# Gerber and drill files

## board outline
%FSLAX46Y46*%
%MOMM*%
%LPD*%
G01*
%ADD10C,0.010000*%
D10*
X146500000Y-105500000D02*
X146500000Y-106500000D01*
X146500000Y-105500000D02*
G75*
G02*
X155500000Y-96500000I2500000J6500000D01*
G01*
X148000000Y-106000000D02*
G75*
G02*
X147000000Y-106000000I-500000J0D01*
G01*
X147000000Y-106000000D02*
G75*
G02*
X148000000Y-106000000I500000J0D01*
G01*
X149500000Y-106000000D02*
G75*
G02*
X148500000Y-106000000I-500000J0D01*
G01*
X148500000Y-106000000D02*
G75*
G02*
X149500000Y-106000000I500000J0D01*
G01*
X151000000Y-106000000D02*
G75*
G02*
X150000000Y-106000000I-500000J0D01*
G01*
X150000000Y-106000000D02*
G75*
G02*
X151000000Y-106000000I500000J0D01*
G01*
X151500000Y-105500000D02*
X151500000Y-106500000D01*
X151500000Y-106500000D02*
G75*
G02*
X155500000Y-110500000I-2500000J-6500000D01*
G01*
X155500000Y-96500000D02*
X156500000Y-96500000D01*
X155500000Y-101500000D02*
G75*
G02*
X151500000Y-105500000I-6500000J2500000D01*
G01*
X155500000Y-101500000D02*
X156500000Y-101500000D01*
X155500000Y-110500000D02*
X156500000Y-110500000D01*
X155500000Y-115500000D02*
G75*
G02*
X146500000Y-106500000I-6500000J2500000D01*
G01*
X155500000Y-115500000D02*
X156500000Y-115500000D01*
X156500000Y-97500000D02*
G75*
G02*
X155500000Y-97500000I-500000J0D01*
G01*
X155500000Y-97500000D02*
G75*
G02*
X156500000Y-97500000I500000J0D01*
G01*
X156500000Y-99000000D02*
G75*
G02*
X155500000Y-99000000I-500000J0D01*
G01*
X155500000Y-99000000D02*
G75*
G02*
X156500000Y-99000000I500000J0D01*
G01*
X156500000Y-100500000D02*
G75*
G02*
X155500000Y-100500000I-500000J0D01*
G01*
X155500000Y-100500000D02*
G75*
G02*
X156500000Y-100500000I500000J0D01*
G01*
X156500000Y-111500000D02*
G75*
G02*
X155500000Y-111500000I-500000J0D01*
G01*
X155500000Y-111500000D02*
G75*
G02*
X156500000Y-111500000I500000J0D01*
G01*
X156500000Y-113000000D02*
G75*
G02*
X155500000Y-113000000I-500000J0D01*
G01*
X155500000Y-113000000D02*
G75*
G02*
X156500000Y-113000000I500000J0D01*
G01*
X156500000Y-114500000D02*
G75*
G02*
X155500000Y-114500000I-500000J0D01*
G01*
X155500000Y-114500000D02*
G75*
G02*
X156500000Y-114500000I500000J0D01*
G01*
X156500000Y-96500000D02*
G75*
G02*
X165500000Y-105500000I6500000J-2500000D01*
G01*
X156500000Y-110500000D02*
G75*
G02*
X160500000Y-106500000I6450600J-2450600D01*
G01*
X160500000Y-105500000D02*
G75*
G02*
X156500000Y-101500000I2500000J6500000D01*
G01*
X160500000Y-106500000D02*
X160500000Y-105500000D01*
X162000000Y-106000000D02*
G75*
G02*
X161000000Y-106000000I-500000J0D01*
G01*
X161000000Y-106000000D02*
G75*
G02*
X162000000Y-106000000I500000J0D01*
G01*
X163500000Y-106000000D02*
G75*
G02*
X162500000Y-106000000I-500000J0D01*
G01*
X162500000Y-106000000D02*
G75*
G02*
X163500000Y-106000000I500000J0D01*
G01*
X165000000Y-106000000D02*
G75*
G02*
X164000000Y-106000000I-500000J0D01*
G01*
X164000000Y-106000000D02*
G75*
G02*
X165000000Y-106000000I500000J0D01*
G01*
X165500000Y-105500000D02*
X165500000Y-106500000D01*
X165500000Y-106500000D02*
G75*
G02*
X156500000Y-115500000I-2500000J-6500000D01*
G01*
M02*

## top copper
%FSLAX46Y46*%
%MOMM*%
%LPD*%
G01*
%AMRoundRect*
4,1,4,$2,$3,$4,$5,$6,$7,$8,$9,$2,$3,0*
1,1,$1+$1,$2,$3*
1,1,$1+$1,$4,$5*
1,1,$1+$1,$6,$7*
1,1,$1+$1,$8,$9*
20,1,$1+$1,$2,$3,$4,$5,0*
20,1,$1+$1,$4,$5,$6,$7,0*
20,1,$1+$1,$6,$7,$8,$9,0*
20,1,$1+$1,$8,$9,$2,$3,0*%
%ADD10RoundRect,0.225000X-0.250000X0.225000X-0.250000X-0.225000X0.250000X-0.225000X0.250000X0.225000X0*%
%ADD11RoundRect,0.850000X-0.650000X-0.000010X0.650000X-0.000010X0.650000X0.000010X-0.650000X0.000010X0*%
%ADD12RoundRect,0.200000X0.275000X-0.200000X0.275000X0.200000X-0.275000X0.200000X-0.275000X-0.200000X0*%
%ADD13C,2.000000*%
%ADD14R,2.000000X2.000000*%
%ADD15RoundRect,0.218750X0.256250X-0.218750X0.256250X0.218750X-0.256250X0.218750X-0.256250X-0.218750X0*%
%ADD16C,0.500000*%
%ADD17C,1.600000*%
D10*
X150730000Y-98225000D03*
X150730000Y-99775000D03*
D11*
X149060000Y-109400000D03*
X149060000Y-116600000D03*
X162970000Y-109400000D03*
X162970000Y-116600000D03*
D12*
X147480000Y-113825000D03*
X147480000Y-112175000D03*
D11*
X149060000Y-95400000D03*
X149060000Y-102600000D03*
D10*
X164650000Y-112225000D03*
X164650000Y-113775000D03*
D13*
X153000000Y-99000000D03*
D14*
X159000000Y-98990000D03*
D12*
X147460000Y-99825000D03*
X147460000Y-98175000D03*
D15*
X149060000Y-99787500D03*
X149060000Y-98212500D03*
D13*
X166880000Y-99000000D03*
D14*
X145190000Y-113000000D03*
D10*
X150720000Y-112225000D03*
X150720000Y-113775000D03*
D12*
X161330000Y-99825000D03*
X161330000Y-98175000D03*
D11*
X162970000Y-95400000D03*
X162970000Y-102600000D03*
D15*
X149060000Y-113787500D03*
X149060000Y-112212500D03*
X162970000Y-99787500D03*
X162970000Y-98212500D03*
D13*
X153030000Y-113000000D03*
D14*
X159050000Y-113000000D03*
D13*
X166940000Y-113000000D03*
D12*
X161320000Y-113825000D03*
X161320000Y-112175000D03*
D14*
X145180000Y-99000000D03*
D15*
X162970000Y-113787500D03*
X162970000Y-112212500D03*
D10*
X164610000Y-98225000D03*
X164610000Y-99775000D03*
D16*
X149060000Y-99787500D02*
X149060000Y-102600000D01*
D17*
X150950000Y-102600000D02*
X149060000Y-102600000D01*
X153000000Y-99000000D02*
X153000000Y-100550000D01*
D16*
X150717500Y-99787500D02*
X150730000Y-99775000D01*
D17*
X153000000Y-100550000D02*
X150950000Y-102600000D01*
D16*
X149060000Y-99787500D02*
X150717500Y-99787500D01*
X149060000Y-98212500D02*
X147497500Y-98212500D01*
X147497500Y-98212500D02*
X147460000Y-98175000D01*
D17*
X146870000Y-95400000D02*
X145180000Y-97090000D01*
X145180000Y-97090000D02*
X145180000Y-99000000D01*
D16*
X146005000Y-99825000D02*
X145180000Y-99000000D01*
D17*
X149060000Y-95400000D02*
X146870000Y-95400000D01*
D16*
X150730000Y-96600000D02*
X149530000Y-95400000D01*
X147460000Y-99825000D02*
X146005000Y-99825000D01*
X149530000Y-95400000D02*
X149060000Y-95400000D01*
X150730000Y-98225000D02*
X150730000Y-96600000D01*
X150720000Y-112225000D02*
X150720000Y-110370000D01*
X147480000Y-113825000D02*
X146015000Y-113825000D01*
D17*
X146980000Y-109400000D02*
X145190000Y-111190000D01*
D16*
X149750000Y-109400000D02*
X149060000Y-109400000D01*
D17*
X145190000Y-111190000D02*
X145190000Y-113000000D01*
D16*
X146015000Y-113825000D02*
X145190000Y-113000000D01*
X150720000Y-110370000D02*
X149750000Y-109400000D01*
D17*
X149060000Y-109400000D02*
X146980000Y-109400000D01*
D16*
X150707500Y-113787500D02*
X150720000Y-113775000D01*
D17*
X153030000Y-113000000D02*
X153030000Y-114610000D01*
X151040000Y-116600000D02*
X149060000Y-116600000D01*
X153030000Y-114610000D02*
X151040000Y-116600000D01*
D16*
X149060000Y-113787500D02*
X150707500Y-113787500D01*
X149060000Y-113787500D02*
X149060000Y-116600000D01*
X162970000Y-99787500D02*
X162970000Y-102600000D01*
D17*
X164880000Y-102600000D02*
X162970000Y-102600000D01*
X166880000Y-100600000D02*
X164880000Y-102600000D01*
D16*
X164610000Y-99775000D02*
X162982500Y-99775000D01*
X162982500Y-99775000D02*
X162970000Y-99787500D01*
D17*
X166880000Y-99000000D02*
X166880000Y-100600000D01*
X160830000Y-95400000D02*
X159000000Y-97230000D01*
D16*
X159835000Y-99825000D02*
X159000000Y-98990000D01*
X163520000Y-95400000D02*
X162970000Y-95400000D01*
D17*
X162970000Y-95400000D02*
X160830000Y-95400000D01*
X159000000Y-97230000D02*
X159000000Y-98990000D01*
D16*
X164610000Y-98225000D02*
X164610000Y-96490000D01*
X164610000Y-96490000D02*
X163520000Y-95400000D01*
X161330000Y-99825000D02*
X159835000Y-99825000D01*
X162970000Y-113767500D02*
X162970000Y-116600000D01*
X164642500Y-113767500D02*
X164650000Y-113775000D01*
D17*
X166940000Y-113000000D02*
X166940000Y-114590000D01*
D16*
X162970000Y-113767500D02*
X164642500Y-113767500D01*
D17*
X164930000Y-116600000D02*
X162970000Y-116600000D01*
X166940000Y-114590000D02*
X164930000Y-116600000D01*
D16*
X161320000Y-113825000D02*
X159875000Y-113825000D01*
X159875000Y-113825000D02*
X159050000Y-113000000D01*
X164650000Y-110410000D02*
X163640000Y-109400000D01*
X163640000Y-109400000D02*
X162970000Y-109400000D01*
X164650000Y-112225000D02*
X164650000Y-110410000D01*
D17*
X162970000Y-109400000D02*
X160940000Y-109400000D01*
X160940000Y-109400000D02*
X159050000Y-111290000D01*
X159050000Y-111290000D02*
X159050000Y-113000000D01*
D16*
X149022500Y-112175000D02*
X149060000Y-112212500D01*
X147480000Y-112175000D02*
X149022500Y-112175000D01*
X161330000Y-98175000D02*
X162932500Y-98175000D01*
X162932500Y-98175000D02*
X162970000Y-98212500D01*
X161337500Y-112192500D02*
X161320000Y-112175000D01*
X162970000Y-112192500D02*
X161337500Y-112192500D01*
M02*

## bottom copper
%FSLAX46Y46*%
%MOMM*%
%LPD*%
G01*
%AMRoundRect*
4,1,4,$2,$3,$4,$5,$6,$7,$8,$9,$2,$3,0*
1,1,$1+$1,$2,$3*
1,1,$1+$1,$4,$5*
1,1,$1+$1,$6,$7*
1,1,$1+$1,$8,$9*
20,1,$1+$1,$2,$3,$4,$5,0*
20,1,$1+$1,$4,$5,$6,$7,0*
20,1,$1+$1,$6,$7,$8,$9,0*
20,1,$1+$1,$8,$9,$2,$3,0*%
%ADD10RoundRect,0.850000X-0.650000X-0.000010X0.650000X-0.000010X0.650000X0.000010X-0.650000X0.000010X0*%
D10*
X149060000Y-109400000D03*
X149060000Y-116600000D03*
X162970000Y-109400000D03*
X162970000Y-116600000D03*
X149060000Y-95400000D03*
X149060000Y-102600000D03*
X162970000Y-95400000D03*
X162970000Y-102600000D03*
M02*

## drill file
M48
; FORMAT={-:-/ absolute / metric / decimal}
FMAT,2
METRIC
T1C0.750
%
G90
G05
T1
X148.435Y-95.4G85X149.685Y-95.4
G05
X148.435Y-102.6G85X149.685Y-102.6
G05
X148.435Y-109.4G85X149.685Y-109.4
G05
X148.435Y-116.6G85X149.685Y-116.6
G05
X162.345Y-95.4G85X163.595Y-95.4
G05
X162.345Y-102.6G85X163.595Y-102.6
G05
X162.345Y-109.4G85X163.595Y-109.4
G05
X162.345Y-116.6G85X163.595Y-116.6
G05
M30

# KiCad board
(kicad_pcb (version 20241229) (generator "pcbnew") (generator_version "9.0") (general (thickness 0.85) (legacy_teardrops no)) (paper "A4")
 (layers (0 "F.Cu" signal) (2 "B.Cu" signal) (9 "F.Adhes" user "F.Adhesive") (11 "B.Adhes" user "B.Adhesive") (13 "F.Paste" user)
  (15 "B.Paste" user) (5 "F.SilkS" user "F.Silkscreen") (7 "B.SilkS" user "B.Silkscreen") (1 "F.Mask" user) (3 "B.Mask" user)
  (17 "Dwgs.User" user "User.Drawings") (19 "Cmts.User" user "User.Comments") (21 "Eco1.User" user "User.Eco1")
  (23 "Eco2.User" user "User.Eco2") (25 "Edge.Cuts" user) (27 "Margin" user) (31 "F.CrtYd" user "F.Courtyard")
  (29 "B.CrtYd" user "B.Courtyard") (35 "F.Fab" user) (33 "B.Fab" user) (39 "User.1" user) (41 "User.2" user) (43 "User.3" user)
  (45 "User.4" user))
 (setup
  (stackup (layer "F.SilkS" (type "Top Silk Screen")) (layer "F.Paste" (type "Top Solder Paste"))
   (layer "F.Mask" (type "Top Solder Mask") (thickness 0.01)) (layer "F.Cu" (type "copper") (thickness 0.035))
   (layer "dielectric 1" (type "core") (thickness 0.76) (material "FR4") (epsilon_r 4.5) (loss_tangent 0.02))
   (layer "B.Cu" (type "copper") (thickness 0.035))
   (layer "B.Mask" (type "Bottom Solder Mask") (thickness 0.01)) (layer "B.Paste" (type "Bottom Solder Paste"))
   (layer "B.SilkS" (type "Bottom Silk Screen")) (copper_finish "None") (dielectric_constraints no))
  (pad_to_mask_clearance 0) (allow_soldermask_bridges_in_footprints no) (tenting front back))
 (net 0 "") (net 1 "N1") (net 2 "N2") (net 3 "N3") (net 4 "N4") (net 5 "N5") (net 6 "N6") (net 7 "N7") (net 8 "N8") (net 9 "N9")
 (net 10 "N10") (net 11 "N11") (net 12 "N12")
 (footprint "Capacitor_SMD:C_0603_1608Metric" (layer "F.Cu") (at 150.73 99 -90)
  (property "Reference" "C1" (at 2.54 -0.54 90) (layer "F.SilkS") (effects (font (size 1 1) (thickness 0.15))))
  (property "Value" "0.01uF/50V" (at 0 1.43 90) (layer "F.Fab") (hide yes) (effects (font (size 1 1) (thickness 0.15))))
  (pad "1" smd roundrect (at -0.775 0 270) (size 0.9 0.95) (layers "F.Cu" "F.Mask" "F.Paste") (roundrect_rratio 0.25) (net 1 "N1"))
  (pad "2" smd roundrect (at 0.775 0 270) (size 0.9 0.95) (layers "F.Cu" "F.Mask" "F.Paste") (roundrect_rratio 0.25) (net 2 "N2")))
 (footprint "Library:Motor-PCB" (layer "F.Cu") (at 149.06 113)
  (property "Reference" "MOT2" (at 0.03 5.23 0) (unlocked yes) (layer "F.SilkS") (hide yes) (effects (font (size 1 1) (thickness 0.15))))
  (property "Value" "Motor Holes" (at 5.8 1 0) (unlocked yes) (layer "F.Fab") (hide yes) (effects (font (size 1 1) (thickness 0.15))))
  (pad "1" thru_hole roundrect (at 0 -3.6) (size 3 1.7) (drill oval 2 0.75) (layers "*.Cu" "*.Mask") (remove_unused_layers no)
   (roundrect_rratio 0.5) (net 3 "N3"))
  (pad "2" thru_hole roundrect (at 0 3.6) (size 3 1.7) (drill oval 2 0.75) (layers "*.Cu" "*.Mask") (remove_unused_layers no)
   (roundrect_rratio 0.5) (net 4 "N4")))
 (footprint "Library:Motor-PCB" (layer "F.Cu") (at 162.97 113)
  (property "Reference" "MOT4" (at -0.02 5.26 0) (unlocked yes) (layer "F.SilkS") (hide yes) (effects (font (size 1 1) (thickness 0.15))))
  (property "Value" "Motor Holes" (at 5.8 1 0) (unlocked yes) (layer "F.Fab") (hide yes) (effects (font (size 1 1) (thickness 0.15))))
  (pad "1" thru_hole roundrect (at 0 -3.6) (size 3 1.7) (drill oval 2 0.75) (layers "*.Cu" "*.Mask") (remove_unused_layers no)
   (roundrect_rratio 0.5) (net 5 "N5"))
  (pad "2" thru_hole roundrect (at 0 3.6) (size 3 1.7) (drill oval 2 0.75) (layers "*.Cu" "*.Mask") (remove_unused_layers no)
   (roundrect_rratio 0.5) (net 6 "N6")))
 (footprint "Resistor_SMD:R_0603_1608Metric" (layer "F.Cu") (at 147.48 113 90)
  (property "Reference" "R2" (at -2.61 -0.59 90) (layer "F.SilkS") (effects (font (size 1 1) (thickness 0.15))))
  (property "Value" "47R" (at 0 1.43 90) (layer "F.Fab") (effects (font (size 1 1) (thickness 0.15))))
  (pad "1" smd roundrect (at -0.825 0 90) (size 0.8 0.95) (layers "F.Cu" "F.Mask" "F.Paste") (roundrect_rratio 0.25) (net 3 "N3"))
  (pad "2" smd roundrect (at 0.825 0 90) (size 0.8 0.95) (layers "F.Cu" "F.Mask" "F.Paste") (roundrect_rratio 0.25) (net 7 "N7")))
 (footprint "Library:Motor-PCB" (layer "F.Cu") (at 149.06 99)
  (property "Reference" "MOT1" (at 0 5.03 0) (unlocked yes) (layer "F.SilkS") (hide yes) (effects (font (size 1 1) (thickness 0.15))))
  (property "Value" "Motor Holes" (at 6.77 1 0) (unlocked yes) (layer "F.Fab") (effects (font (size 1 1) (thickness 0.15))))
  (pad "1" thru_hole roundrect (at 0 -3.6) (size 3 1.7) (drill oval 2 0.75) (layers "*.Cu" "*.Mask") (remove_unused_layers no)
   (roundrect_rratio 0.5) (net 1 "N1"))
  (pad "2" thru_hole roundrect (at 0 3.6) (size 3 1.7) (drill oval 2 0.75) (layers "*.Cu" "*.Mask") (remove_unused_layers no)
   (roundrect_rratio 0.5) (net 2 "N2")))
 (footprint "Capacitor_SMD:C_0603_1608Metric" (layer "F.Cu") (at 164.65 113 -90)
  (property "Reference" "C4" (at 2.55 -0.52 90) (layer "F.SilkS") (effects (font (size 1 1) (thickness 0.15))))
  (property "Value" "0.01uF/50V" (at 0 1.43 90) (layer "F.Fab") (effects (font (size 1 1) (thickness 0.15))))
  (pad "1" smd roundrect (at -0.775 0 270) (size 0.9 0.95) (layers "F.Cu" "F.Mask" "F.Paste") (roundrect_rratio 0.25) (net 5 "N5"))
  (pad "2" smd roundrect (at 0.775 0 270) (size 0.9 0.95) (layers "F.Cu" "F.Mask" "F.Paste") (roundrect_rratio 0.25) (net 6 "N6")))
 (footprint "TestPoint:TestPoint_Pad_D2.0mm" (layer "F.Cu") (at 153 99)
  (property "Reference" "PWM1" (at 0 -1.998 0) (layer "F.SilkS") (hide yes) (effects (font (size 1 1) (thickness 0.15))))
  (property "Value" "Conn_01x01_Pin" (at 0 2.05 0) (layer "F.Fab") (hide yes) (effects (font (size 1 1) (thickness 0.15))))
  (pad "1" smd circle (at 0 0) (size 2 2) (layers "F.Cu" "F.Mask") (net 2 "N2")))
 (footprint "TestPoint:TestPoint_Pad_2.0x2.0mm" (layer "F.Cu") (at 159 98.99)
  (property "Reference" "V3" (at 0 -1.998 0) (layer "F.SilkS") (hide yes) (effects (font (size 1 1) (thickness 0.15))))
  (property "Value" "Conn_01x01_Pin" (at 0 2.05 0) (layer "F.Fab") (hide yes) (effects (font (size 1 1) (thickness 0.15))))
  (pad "1" smd rect (at 0 0) (size 2 2) (layers "F.Cu" "F.Mask") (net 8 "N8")))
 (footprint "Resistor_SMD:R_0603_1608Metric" (layer "F.Cu") (at 147.46 99 90)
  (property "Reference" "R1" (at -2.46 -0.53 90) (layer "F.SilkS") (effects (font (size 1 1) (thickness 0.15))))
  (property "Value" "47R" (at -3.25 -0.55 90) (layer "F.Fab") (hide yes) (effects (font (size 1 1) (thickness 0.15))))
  (pad "1" smd roundrect (at -0.825 0 90) (size 0.8 0.95) (layers "F.Cu" "F.Mask" "F.Paste") (roundrect_rratio 0.25) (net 1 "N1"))
  (pad "2" smd roundrect (at 0.825 0 90) (size 0.8 0.95) (layers "F.Cu" "F.Mask" "F.Paste") (roundrect_rratio 0.25) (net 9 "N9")))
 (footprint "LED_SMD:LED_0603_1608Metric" (layer "F.Cu") (at 149.06 99 90)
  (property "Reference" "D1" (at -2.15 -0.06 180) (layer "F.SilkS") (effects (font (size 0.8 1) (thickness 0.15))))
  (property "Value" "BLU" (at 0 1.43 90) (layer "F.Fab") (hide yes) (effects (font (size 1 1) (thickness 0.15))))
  (pad "1" smd roundrect (at -0.7875 0 90) (size 0.875 0.95) (layers "F.Cu" "F.Mask" "F.Paste") (roundrect_rratio 0.25) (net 2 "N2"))
  (pad "2" smd roundrect (at 0.7875 0 90) (size 0.875 0.95) (layers "F.Cu" "F.Mask" "F.Paste") (roundrect_rratio 0.25) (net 9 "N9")))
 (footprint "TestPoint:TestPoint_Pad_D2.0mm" (layer "F.Cu") (at 166.88 99 90)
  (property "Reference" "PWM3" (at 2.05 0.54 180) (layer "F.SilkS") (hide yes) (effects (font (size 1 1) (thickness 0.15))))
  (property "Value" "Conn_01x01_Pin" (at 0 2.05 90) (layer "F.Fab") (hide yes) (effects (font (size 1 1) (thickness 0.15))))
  (pad "1" smd circle (at 0 0 90) (size 2 2) (layers "F.Cu" "F.Mask") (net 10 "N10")))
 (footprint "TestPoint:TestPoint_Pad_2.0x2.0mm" (layer "F.Cu") (at 145.19 113)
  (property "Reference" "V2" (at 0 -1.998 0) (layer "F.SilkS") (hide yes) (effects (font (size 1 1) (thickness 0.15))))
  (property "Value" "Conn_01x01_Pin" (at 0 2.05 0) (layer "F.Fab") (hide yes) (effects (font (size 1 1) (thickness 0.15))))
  (pad "1" smd rect (at 0 0) (size 2 2) (layers "F.Cu" "F.Mask") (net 3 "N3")))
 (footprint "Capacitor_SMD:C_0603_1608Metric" (layer "F.Cu") (at 150.72 113 -90)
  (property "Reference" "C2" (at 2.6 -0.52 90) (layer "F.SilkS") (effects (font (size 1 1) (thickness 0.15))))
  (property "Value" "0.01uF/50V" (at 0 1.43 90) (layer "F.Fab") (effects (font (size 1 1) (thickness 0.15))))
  (pad "1" smd roundrect (at -0.775 0 270) (size 0.9 0.95) (layers "F.Cu" "F.Mask" "F.Paste") (roundrect_rratio 0.25) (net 3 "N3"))
  (pad "2" smd roundrect (at 0.775 0 270) (size 0.9 0.95) (layers "F.Cu" "F.Mask" "F.Paste") (roundrect_rratio 0.25) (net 4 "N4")))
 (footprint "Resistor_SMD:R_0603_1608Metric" (layer "F.Cu") (at 161.33 99 90)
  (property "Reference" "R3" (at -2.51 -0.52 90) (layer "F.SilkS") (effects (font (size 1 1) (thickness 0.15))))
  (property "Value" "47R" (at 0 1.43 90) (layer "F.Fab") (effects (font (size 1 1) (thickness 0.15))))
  (pad "1" smd roundrect (at -0.825 0 90) (size 0.8 0.95) (layers "F.Cu" "F.Mask" "F.Paste") (roundrect_rratio 0.25) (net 8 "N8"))
  (pad "2" smd roundrect (at 0.825 0 90) (size 0.8 0.95) (layers "F.Cu" "F.Mask" "F.Paste") (roundrect_rratio 0.25) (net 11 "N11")))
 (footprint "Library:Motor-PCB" (layer "F.Cu") (at 162.97 99)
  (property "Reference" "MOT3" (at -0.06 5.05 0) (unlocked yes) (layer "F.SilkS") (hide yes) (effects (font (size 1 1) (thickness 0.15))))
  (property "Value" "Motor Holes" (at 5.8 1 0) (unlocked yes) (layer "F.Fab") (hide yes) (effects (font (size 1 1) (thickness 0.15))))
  (pad "1" thru_hole roundrect (at 0 -3.6) (size 3 1.7) (drill oval 2 0.75) (layers "*.Cu" "*.Mask") (remove_unused_layers no)
   (roundrect_rratio 0.5) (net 8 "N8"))
  (pad "2" thru_hole roundrect (at 0 3.6) (size 3 1.7) (drill oval 2 0.75) (layers "*.Cu" "*.Mask") (remove_unused_layers no)
   (roundrect_rratio 0.5) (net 10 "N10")))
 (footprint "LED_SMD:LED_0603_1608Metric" (layer "F.Cu") (at 149.06 113 90)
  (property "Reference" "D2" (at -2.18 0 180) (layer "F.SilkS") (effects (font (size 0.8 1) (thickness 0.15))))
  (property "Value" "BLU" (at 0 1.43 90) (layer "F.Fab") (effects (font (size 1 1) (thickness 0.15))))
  (pad "1" smd roundrect (at -0.7875 0 90) (size 0.875 0.95) (layers "F.Cu" "F.Mask" "F.Paste") (roundrect_rratio 0.25) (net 4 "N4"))
  (pad "2" smd roundrect (at 0.7875 0 90) (size 0.875 0.95) (layers "F.Cu" "F.Mask" "F.Paste") (roundrect_rratio 0.25) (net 7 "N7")))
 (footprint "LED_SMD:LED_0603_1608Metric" (layer "F.Cu") (at 162.97 99 90)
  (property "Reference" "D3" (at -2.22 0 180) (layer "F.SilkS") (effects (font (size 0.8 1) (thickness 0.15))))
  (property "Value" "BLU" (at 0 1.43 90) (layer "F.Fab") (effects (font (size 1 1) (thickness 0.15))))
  (pad "1" smd roundrect (at -0.7875 0 90) (size 0.875 0.95) (layers "F.Cu" "F.Mask" "F.Paste") (roundrect_rratio 0.25) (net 10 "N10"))
  (pad "2" smd roundrect (at 0.7875 0 90) (size 0.875 0.95) (layers "F.Cu" "F.Mask" "F.Paste") (roundrect_rratio 0.25) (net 11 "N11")))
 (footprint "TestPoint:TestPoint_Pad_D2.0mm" (layer "F.Cu") (at 153.03 113)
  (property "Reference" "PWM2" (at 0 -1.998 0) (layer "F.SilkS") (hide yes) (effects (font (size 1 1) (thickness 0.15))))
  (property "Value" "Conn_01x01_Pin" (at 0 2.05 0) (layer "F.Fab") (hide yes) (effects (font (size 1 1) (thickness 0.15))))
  (pad "1" smd circle (at 0 0) (size 2 2) (layers "F.Cu" "F.Mask") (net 4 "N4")))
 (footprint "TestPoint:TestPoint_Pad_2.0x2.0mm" (layer "F.Cu") (at 159.05 113)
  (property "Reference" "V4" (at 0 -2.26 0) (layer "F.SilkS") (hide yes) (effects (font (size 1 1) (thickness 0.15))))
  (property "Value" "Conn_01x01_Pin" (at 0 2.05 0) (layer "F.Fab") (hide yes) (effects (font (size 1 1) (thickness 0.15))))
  (pad "1" smd rect (at 0 0) (size 2 2) (layers "F.Cu" "F.Mask") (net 5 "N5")))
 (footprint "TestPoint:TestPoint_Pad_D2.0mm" (layer "F.Cu") (at 166.94 113)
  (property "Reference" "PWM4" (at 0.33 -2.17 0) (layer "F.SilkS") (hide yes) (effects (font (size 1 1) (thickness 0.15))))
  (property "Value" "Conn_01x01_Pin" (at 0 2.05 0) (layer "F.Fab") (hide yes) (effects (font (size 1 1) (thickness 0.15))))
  (pad "1" smd circle (at 0 0) (size 2 2) (layers "F.Cu" "F.Mask") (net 6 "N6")))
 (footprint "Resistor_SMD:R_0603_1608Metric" (layer "F.Cu") (at 161.32 113 90)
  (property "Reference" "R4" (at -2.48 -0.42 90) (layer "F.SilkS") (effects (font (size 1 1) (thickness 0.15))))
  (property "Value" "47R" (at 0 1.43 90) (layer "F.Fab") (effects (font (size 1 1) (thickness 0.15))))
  (pad "1" smd roundrect (at -0.825 0 90) (size 0.8 0.95) (layers "F.Cu" "F.Mask" "F.Paste") (roundrect_rratio 0.25) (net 5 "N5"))
  (pad "2" smd roundrect (at 0.825 0 90) (size 0.8 0.95) (layers "F.Cu" "F.Mask" "F.Paste") (roundrect_rratio 0.25) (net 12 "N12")))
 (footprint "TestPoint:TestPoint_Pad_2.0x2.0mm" (layer "F.Cu") (at 145.18 99)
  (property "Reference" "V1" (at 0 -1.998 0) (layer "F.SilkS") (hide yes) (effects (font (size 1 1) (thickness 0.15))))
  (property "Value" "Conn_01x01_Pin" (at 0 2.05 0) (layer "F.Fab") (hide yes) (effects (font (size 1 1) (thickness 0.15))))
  (pad "1" smd rect (at 0 0) (size 2 2) (layers "F.Cu" "F.Mask") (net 1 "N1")))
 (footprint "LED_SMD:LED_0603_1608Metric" (layer "F.Cu") (at 162.97 113 90)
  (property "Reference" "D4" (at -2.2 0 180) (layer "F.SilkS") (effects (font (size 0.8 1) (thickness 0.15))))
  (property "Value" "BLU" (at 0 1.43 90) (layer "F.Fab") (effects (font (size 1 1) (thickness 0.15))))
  (pad "1" smd roundrect (at -0.7875 0 90) (size 0.875 0.95) (layers "F.Cu" "F.Mask" "F.Paste") (roundrect_rratio 0.25) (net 6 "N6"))
  (pad "2" smd roundrect (at 0.7875 0 90) (size 0.875 0.95) (layers "F.Cu" "F.Mask" "F.Paste") (roundrect_rratio 0.25) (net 12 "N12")))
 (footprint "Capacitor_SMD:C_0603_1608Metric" (layer "F.Cu") (at 164.61 99 -90)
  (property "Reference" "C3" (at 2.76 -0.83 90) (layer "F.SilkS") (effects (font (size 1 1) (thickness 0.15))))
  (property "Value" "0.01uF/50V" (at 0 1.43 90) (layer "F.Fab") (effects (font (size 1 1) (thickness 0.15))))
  (pad "1" smd roundrect (at -0.775 0 270) (size 0.9 0.95) (layers "F.Cu" "F.Mask" "F.Paste") (roundrect_rratio 0.25) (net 8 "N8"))
  (pad "2" smd roundrect (at 0.775 0 270) (size 0.9 0.95) (layers "F.Cu" "F.Mask" "F.Paste") (roundrect_rratio 0.25) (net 10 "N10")))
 (gr_line (start 146.5 105.5) (end 146.5 106.5) (stroke (width 0.01) (type solid)) (layer "Edge.Cuts"))
 (gr_arc (start 146.5 105.5) (mid 144.075571 94.075571) (end 155.5 96.5) (stroke (width 0.01) (type solid)) (layer "Edge.Cuts"))
 (gr_circle (center 147.5 106) (end 147.5 105.5) (stroke (width 0.01) (type solid)) (fill no) (layer "Edge.Cuts"))
 (gr_circle (center 149 106) (end 149 105.5) (stroke (width 0.01) (type solid)) (fill no) (layer "Edge.Cuts"))
 (gr_circle (center 150.5 106) (end 150.5 105.5) (stroke (width 0.01) (type solid)) (fill no) (layer "Edge.Cuts"))
 (gr_line (start 151.5 105.5) (end 151.5 106.5) (stroke (width 0.01) (type solid)) (layer "Edge.Cuts"))
 (gr_arc (start 151.5 106.5) (mid 153.924429 108.075571) (end 155.5 110.5) (stroke (width 0.01) (type solid)) (layer "Edge.Cuts"))
 (gr_line (start 155.5 96.5) (end 156.5 96.5) (stroke (width 0.01) (type solid)) (layer "Edge.Cuts"))
 (gr_arc (start 155.5 101.5) (mid 153.924429 103.924429) (end 151.5 105.5) (stroke (width 0.01) (type solid)) (layer "Edge.Cuts"))
 (gr_line (start 155.5 101.5) (end 156.5 101.5) (stroke (width 0.01) (type solid)) (layer "Edge.Cuts"))
 (gr_line (start 155.5 110.5) (end 156.5 110.5) (stroke (width 0.01) (type solid)) (layer "Edge.Cuts"))
 (gr_arc (start 155.5 115.5) (mid 144.075571 117.924429) (end 146.5 106.5) (stroke (width 0.01) (type solid)) (layer "Edge.Cuts"))
 (gr_line (start 155.5 115.5) (end 156.5 115.5) (stroke (width 0.01) (type solid)) (layer "Edge.Cuts"))
 (gr_circle (center 156 97.5) (end 155.5 97.5) (stroke (width 0.01) (type solid)) (fill no) (layer "Edge.Cuts"))
 (gr_circle (center 156 99) (end 155.5 99) (stroke (width 0.01) (type solid)) (fill no) (layer "Edge.Cuts"))
 (gr_circle (center 156 100.5) (end 155.5 100.5) (stroke (width 0.01) (type solid)) (fill no) (layer "Edge.Cuts"))
 (gr_circle (center 156 111.5) (end 155.5 111.5) (stroke (width 0.01) (type solid)) (fill no) (layer "Edge.Cuts"))
 (gr_circle (center 156 113) (end 155.5 113) (stroke (width 0.01) (type solid)) (fill no) (layer "Edge.Cuts"))
 (gr_circle (center 156 114.5) (end 155.5 114.5) (stroke (width 0.01) (type solid)) (fill no) (layer "Edge.Cuts"))
 (gr_arc (start 156.5 96.5) (mid 167.924429 94.075571) (end 165.5 105.5) (stroke (width 0.01) (type solid)) (layer "Edge.Cuts"))
 (gr_arc (start 156.5 110.5) (mid 158.072271 108.070282) (end 160.5 106.5) (stroke (width 0.01) (type solid)) (layer "Edge.Cuts"))
 (gr_arc (start 160.5 105.5) (mid 158.075571 103.924429) (end 156.5 101.5) (stroke (width 0.01) (type solid)) (layer "Edge.Cuts"))
 (gr_line (start 160.5 106.5) (end 160.5 105.5) (stroke (width 0.01) (type solid)) (layer "Edge.Cuts"))
 (gr_circle (center 161.5 106) (end 161.5 105.5) (stroke (width 0.01) (type solid)) (fill no) (layer "Edge.Cuts"))
 (gr_circle (center 163 106) (end 163 105.5) (stroke (width 0.01) (type solid)) (fill no) (layer "Edge.Cuts"))
 (gr_circle (center 164.5 106) (end 164.5 105.5) (stroke (width 0.01) (type solid)) (fill no) (layer "Edge.Cuts"))
 (gr_line (start 165.5 105.5) (end 165.5 106.5) (stroke (width 0.01) (type solid)) (layer "Edge.Cuts"))
 (gr_arc (start 165.5 106.5) (mid 167.924429 117.924429) (end 156.5 115.5) (stroke (width 0.01) (type solid)) (layer "Edge.Cuts"))
 (segment (start 149.06 99.7875) (end 149.06 102.6) (width 0.5) (layer "F.Cu") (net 2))
 (segment (start 150.95 102.6) (end 149.06 102.6) (width 1.6) (layer "F.Cu") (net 2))
 (segment (start 153 99) (end 153 100.55) (width 1.6) (layer "F.Cu") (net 2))
 (segment (start 150.7175 99.7875) (end 150.73 99.775) (width 0.5) (layer "F.Cu") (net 2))
 (segment (start 153 100.55) (end 150.95 102.6) (width 1.6) (layer "F.Cu") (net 2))
 (segment (start 149.06 99.7875) (end 150.7175 99.7875) (width 0.5) (layer "F.Cu") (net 2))
 (segment (start 149.06 98.2125) (end 147.4975 98.2125) (width 0.5) (layer "F.Cu") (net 9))
 (segment (start 147.4975 98.2125) (end 147.46 98.175) (width 0.5) (layer "F.Cu") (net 9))
 (segment (start 146.87 95.4) (end 145.18 97.09) (width 1.6) (layer "F.Cu") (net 1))
 (segment (start 145.18 97.09) (end 145.18 99) (width 1.6) (layer "F.Cu") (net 1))
 (segment (start 146.005 99.825) (end 145.18 99) (width 0.5) (layer "F.Cu") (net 1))
 (segment (start 149.06 95.4) (end 146.87 95.4) (width 1.6) (layer "F.Cu") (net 1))
 (segment (start 150.73 96.6) (end 149.53 95.4) (width 0.5) (layer "F.Cu") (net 1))
 (segment (start 147.46 99.825) (end 146.005 99.825) (width 0.5) (layer "F.Cu") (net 1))
 (segment (start 149.53 95.4) (end 149.06 95.4) (width 0.5) (layer "F.Cu") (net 1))
 (segment (start 150.73 98.225) (end 150.73 96.6) (width 0.5) (layer "F.Cu") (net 1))
 (segment (start 150.72 112.225) (end 150.72 110.37) (width 0.5) (layer "F.Cu") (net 3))
 (segment (start 147.48 113.825) (end 146.015 113.825) (width 0.5) (layer "F.Cu") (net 3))
 (segment (start 146.98 109.4) (end 145.19 111.19) (width 1.6) (layer "F.Cu") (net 3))
 (segment (start 149.75 109.4) (end 149.06 109.4) (width 0.5) (layer "F.Cu") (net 3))
 (segment (start 145.19 111.19) (end 145.19 113) (width 1.6) (layer "F.Cu") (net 3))
 (segment (start 146.015 113.825) (end 145.19 113) (width 0.5) (layer "F.Cu") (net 3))
 (segment (start 150.72 110.37) (end 149.75 109.4) (width 0.5) (layer "F.Cu") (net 3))
 (segment (start 149.06 109.4) (end 146.98 109.4) (width 1.6) (layer "F.Cu") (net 3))
 (segment (start 150.7075 113.7875) (end 150.72 113.775) (width 0.5) (layer "F.Cu") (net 4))
 (segment (start 153.03 113) (end 153.03 114.61) (width 1.6) (layer "F.Cu") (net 4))
 (segment (start 151.04 116.6) (end 149.06 116.6) (width 1.6) (layer "F.Cu") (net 4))
 (segment (start 153.03 114.61) (end 151.04 116.6) (width 1.6) (layer "F.Cu") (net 4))
 (segment (start 149.06 113.7875) (end 150.7075 113.7875) (width 0.5) (layer "F.Cu") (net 4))
 (segment (start 149.06 113.7875) (end 149.06 116.6) (width 0.5) (layer "F.Cu") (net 4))
 (segment (start 162.97 99.7875) (end 162.97 102.6) (width 0.5) (layer "F.Cu") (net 10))
 (segment (start 164.88 102.6) (end 162.97 102.6) (width 1.6) (layer "F.Cu") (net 10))
 (segment (start 166.88 100.6) (end 164.88 102.6) (width 1.6) (layer "F.Cu") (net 10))
 (segment (start 164.61 99.775) (end 162.9825 99.775) (width 0.5) (layer "F.Cu") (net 10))
 (segment (start 162.9825 99.775) (end 162.97 99.7875) (width 0.5) (layer "F.Cu") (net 10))
 (segment (start 166.88 99) (end 166.88 100.6) (width 1.6) (layer "F.Cu") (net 10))
 (segment (start 160.83 95.4) (end 159 97.23) (width 1.6) (layer "F.Cu") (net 8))
 (segment (start 159.835 99.825) (end 159 98.99) (width 0.5) (layer "F.Cu") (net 8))
 (segment (start 163.52 95.4) (end 162.97 95.4) (width 0.5) (layer "F.Cu") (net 8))
 (segment (start 162.97 95.4) (end 160.83 95.4) (width 1.6) (layer "F.Cu") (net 8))
 (segment (start 159 97.23) (end 159 98.99) (width 1.6) (layer "F.Cu") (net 8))
 (segment (start 164.61 98.225) (end 164.61 96.49) (width 0.5) (layer "F.Cu") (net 8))
 (segment (start 164.61 96.49) (end 163.52 95.4) (width 0.5) (layer "F.Cu") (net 8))
 (segment (start 161.33 99.825) (end 159.835 99.825) (width 0.5) (layer "F.Cu") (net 8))
 (segment (start 162.97 113.7675) (end 162.97 116.6) (width 0.5) (layer "F.Cu") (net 6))
 (segment (start 164.6425 113.7675) (end 164.65 113.775) (width 0.5) (layer "F.Cu") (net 6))
 (segment (start 166.94 113) (end 166.94 114.59) (width 1.6) (layer "F.Cu") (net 6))
 (segment (start 162.97 113.7675) (end 164.6425 113.7675) (width 0.5) (layer "F.Cu") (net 6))
 (segment (start 164.93 116.6) (end 162.97 116.6) (width 1.6) (layer "F.Cu") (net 6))
 (segment (start 166.94 114.59) (end 164.93 116.6) (width 1.6) (layer "F.Cu") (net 6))
 (segment (start 161.32 113.825) (end 159.875 113.825) (width 0.5) (layer "F.Cu") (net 5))
 (segment (start 159.875 113.825) (end 159.05 113) (width 0.5) (layer "F.Cu") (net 5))
 (segment (start 164.65 110.41) (end 163.64 109.4) (width 0.5) (layer "F.Cu") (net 5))
 (segment (start 163.64 109.4) (end 162.97 109.4) (width 0.5) (layer "F.Cu") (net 5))
 (segment (start 164.65 112.225) (end 164.65 110.41) (width 0.5) (layer "F.Cu") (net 5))
 (segment (start 162.97 109.4) (end 160.94 109.4) (width 1.6) (layer "F.Cu") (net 5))
 (segment (start 160.94 109.4) (end 159.05 111.29) (width 1.6) (layer "F.Cu") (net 5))
 (segment (start 159.05 111.29) (end 159.05 113) (width 1.6) (layer "F.Cu") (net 5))
 (segment (start 149.0225 112.175) (end 149.06 112.2125) (width 0.5) (layer "F.Cu") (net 7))
 (segment (start 147.48 112.175) (end 149.0225 112.175) (width 0.5) (layer "F.Cu") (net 7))
 (segment (start 161.33 98.175) (end 162.9325 98.175) (width 0.5) (layer "F.Cu") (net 11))
 (segment (start 162.9325 98.175) (end 162.97 98.2125) (width 0.5) (layer "F.Cu") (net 11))
 (segment (start 161.3375 112.1925) (end 161.32 112.175) (width 0.5) (layer "F.Cu") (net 12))
 (segment (start 162.97 112.1925) (end 161.3375 112.1925) (width 0.5) (layer "F.Cu") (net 12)))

